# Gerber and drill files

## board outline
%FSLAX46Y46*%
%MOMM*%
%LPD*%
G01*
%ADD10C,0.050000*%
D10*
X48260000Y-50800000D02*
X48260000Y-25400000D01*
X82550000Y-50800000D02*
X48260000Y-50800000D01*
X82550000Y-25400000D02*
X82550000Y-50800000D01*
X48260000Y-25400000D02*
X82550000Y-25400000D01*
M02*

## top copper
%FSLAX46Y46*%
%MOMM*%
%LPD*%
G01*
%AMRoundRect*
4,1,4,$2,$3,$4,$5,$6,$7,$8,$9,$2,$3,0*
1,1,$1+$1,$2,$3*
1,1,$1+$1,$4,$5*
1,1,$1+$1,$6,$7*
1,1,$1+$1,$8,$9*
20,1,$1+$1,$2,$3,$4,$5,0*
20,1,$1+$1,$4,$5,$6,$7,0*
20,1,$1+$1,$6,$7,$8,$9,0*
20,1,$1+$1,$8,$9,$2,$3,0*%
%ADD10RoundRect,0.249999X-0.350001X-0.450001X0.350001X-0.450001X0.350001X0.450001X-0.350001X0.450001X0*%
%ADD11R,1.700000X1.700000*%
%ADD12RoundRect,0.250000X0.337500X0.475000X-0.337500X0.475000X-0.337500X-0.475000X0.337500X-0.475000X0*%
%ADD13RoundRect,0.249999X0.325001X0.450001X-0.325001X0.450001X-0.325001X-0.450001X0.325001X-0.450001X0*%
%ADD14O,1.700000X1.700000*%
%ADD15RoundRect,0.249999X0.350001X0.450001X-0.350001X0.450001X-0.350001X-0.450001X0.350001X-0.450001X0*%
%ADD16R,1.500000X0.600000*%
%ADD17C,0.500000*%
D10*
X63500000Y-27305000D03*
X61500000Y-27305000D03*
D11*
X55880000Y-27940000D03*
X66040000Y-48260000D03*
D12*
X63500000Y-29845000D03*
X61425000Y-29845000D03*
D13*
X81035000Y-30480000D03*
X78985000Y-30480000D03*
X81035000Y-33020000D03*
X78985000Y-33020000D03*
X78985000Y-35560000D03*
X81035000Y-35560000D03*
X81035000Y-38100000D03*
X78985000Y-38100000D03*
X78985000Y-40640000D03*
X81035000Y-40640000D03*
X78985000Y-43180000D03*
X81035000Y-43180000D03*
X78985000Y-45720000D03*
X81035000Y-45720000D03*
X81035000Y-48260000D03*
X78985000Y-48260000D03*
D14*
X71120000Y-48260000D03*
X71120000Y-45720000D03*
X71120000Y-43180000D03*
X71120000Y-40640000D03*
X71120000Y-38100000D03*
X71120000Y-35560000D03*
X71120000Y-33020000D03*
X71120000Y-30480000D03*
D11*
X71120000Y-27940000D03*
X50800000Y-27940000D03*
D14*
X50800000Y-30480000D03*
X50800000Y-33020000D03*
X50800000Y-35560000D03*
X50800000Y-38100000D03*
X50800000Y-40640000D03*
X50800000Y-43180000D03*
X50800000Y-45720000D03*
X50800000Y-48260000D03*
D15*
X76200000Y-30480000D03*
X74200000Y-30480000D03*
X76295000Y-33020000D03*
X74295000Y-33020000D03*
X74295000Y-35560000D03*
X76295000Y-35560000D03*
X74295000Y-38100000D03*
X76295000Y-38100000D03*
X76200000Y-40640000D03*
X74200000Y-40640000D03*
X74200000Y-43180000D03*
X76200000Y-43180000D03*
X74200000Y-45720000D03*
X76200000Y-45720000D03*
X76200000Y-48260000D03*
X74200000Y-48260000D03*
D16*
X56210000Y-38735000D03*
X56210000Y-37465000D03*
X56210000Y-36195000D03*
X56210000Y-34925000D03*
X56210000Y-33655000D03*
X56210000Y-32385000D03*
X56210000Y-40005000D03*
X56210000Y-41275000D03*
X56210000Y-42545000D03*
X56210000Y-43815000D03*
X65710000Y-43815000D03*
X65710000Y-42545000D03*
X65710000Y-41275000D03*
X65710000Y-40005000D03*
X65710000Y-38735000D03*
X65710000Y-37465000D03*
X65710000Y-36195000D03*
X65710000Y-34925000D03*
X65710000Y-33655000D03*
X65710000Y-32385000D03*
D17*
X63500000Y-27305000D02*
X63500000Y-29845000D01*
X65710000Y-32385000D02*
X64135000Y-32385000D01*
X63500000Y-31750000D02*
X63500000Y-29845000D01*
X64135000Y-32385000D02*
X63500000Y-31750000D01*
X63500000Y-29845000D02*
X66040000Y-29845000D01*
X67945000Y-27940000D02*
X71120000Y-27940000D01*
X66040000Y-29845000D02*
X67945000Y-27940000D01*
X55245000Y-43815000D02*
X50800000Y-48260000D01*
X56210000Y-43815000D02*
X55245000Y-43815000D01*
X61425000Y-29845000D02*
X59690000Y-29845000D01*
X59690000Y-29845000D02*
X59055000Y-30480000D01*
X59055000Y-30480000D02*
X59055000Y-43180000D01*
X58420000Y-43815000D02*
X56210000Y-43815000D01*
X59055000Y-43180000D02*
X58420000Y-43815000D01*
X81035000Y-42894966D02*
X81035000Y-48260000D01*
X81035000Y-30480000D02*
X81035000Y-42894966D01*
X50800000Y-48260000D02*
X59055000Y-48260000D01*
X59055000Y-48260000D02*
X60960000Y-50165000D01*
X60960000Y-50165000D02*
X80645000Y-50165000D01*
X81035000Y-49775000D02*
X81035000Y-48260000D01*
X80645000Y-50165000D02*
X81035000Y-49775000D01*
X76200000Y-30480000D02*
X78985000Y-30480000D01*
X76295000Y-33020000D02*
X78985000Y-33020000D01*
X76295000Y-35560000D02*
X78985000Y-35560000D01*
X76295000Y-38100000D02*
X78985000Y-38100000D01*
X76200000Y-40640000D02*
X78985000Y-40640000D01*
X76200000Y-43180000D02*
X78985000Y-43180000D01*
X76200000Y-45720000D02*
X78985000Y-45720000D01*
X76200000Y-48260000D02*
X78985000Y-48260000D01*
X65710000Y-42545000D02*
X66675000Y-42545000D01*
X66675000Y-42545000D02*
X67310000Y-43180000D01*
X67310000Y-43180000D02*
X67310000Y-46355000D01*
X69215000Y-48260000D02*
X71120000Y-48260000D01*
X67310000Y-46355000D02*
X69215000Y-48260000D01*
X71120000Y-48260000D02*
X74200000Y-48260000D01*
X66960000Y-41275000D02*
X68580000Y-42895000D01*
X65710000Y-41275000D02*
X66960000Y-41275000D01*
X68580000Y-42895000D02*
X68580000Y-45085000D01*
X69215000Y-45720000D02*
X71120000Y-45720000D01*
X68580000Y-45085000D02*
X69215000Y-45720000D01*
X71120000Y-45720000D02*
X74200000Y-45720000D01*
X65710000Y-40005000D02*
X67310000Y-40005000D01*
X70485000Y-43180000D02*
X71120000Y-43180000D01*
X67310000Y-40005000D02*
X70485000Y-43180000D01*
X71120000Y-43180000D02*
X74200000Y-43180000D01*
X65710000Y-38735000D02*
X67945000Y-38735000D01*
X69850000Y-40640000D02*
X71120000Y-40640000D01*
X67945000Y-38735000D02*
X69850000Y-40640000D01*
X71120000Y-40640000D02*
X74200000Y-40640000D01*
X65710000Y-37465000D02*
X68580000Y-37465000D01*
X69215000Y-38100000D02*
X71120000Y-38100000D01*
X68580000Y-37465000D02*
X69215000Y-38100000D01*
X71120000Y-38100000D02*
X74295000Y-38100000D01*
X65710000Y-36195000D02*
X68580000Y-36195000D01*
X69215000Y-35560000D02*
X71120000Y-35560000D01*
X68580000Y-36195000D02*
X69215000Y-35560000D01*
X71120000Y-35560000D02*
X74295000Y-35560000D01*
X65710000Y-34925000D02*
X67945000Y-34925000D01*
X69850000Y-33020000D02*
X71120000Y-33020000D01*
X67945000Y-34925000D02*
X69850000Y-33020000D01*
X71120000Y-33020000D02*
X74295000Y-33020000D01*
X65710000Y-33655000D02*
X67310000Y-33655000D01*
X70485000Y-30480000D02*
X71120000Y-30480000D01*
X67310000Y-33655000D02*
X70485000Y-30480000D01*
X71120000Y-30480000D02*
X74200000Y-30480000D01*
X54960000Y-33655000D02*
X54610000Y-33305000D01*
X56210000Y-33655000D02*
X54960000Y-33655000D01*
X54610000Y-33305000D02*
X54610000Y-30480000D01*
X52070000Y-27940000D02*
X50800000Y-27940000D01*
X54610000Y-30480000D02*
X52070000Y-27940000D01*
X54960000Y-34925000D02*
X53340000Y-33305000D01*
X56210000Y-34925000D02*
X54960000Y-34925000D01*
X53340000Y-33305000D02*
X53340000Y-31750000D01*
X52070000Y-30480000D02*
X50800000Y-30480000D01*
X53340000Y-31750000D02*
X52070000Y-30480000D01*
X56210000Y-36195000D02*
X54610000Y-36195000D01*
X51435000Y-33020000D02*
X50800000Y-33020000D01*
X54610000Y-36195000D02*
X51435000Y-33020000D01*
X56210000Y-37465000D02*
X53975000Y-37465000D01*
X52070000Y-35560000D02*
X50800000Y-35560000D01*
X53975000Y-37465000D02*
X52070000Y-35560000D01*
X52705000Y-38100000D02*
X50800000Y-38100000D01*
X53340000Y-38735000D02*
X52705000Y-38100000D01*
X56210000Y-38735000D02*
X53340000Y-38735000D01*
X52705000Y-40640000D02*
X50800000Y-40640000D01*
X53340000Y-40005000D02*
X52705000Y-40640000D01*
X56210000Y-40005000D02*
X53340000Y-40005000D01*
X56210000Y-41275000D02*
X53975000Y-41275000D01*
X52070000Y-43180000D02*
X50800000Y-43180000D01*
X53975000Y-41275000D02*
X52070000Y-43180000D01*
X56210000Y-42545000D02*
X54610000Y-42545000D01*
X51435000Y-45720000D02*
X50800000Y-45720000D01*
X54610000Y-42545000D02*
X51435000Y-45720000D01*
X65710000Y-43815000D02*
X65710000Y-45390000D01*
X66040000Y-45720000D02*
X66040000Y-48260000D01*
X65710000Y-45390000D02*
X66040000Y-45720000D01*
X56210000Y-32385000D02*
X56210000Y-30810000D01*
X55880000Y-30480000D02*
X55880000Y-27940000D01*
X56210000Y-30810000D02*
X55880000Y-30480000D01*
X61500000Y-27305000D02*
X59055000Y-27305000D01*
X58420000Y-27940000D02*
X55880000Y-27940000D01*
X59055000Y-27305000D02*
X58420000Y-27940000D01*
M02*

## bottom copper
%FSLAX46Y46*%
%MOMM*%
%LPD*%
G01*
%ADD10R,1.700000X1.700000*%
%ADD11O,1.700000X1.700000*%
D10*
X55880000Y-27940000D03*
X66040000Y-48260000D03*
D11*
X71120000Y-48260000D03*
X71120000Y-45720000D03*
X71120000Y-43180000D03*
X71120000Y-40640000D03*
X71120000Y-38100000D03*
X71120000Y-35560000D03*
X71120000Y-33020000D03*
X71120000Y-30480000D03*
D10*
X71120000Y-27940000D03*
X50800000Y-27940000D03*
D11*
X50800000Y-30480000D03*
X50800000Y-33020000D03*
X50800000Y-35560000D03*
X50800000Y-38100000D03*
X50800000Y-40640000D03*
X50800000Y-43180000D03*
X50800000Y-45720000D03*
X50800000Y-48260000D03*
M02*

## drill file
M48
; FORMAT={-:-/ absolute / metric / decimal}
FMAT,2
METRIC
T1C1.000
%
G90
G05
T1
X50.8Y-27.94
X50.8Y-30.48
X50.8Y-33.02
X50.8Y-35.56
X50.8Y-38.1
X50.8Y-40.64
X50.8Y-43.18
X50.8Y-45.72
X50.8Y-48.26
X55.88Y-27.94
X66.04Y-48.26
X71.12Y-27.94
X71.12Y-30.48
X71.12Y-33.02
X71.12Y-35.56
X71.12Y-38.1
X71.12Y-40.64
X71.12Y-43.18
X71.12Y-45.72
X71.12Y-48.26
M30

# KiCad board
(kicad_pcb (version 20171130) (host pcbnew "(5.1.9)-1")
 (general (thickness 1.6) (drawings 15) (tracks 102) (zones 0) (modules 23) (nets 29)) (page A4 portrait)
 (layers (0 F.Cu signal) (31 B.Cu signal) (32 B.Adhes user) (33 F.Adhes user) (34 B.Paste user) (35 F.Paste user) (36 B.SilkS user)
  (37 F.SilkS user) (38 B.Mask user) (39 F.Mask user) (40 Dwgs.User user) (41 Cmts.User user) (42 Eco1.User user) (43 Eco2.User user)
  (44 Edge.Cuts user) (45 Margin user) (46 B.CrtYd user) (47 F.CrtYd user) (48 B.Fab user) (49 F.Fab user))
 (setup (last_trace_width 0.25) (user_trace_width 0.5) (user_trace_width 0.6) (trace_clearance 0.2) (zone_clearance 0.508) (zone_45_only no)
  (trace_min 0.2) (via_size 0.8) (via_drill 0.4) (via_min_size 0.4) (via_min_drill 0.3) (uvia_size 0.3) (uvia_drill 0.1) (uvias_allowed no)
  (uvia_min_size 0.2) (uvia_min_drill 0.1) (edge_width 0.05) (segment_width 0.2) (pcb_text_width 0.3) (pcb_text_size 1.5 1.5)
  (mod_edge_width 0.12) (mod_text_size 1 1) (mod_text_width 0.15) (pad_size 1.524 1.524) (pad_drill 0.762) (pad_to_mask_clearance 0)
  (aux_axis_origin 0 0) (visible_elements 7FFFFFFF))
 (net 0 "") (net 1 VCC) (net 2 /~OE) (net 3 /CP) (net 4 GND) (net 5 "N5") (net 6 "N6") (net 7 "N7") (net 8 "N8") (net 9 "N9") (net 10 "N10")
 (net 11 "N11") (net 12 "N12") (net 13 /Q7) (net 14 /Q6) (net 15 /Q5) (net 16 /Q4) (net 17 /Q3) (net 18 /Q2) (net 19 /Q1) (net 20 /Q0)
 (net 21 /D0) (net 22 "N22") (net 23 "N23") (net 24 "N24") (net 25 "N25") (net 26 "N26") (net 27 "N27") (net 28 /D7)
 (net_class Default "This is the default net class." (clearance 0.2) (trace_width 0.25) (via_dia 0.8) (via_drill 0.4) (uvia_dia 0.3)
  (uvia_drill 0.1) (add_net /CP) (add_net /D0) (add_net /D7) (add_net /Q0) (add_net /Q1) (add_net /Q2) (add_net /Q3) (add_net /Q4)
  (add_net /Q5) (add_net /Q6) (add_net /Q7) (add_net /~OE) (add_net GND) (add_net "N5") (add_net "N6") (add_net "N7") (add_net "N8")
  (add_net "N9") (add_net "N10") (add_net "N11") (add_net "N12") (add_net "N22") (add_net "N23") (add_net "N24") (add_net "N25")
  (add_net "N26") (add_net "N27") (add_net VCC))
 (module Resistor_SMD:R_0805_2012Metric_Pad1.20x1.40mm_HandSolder (layer F.Cu) (at 62.5 27.305)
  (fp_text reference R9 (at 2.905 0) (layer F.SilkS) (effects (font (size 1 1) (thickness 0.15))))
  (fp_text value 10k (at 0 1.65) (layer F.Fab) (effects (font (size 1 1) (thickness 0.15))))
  (pad 2 smd roundrect (at 1 0) (size 1.2 1.4) (layers F.Cu F.Paste F.Mask) (roundrect_rratio 0.2083325) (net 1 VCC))
  (pad 1 smd roundrect (at -1 0) (size 1.2 1.4) (layers F.Cu F.Paste F.Mask) (roundrect_rratio 0.2083325) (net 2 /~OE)))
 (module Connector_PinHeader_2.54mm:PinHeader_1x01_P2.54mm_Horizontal (layer F.Cu) (at 55.88 27.94 90)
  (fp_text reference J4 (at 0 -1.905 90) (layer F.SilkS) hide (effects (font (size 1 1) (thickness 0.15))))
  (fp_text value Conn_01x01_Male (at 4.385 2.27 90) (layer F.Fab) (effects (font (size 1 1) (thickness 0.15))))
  (pad 1 thru_hole rect (at 0 0 90) (size 1.7 1.7) (drill 1) (layers *.Cu *.Mask) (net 2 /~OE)))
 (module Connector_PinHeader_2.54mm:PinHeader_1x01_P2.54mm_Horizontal (layer F.Cu) (at 66.04 48.26 270)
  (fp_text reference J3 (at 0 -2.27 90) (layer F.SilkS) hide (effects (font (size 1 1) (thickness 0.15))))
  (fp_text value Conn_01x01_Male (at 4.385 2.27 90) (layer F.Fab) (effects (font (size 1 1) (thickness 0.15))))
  (pad 1 thru_hole rect (at 0 0 270) (size 1.7 1.7) (drill 1) (layers *.Cu *.Mask) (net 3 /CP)))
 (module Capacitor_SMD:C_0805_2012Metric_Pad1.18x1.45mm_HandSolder (layer F.Cu) (at 62.4625 29.845 180)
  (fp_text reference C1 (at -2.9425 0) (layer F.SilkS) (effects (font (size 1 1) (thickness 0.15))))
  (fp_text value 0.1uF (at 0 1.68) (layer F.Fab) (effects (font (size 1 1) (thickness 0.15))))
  (pad 1 smd roundrect (at -1.0375 0 180) (size 1.175 1.45) (layers F.Cu F.Paste F.Mask) (roundrect_rratio 0.2127659574468085) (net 1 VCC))
  (pad 2 smd roundrect (at 1.0375 0 180) (size 1.175 1.45) (layers F.Cu F.Paste F.Mask) (roundrect_rratio 0.2127659574468085) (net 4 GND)))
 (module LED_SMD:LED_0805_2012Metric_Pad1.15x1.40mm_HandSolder (layer F.Cu) (at 80.01 30.48 180)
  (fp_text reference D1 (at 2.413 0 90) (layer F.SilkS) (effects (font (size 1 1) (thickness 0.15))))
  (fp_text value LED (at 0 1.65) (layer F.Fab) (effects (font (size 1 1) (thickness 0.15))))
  (pad 1 smd roundrect (at -1.025 0 180) (size 1.15 1.4) (layers F.Cu F.Paste F.Mask) (roundrect_rratio 0.2173904347826087) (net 4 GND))
  (pad 2 smd roundrect (at 1.025 0 180) (size 1.15 1.4) (layers F.Cu F.Paste F.Mask) (roundrect_rratio 0.2173904347826087) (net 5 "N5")))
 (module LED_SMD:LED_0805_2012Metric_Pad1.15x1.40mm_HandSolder (layer F.Cu) (at 80.01 33.02 180)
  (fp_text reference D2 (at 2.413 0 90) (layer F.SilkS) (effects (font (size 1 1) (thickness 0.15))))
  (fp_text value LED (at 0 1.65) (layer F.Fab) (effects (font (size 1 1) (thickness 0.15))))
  (pad 1 smd roundrect (at -1.025 0 180) (size 1.15 1.4) (layers F.Cu F.Paste F.Mask) (roundrect_rratio 0.2173904347826087) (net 4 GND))
  (pad 2 smd roundrect (at 1.025 0 180) (size 1.15 1.4) (layers F.Cu F.Paste F.Mask) (roundrect_rratio 0.2173904347826087) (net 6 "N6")))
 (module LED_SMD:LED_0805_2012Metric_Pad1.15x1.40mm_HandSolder (layer F.Cu) (at 80.01 35.56 180)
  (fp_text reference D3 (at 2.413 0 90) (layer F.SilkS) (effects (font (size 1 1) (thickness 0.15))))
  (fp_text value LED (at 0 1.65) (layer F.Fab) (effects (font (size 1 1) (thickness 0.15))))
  (pad 2 smd roundrect (at 1.025 0 180) (size 1.15 1.4) (layers F.Cu F.Paste F.Mask) (roundrect_rratio 0.2173904347826087) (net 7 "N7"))
  (pad 1 smd roundrect (at -1.025 0 180) (size 1.15 1.4) (layers F.Cu F.Paste F.Mask) (roundrect_rratio 0.2173904347826087) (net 4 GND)))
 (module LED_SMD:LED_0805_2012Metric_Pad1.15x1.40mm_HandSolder (layer F.Cu) (at 80.01 38.1 180)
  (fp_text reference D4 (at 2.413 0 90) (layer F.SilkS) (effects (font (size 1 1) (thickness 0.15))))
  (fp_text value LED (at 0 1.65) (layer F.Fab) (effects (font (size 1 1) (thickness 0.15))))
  (pad 1 smd roundrect (at -1.025 0 180) (size 1.15 1.4) (layers F.Cu F.Paste F.Mask) (roundrect_rratio 0.2173904347826087) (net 4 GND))
  (pad 2 smd roundrect (at 1.025 0 180) (size 1.15 1.4) (layers F.Cu F.Paste F.Mask) (roundrect_rratio 0.2173904347826087) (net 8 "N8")))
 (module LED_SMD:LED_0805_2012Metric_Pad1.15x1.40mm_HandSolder (layer F.Cu) (at 80.01 40.64 180)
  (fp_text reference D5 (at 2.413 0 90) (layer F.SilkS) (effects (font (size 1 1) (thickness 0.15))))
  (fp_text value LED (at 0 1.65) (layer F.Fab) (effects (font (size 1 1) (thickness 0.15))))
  (pad 2 smd roundrect (at 1.025 0 180) (size 1.15 1.4) (layers F.Cu F.Paste F.Mask) (roundrect_rratio 0.2173904347826087) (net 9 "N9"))
  (pad 1 smd roundrect (at -1.025 0 180) (size 1.15 1.4) (layers F.Cu F.Paste F.Mask) (roundrect_rratio 0.2173904347826087) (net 4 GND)))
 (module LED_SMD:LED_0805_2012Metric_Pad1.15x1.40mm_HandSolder (layer F.Cu) (at 80.01 43.18 180)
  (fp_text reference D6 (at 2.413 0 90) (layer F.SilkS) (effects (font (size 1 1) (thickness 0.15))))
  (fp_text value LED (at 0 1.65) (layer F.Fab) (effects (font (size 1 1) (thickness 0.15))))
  (pad 2 smd roundrect (at 1.025 0 180) (size 1.15 1.4) (layers F.Cu F.Paste F.Mask) (roundrect_rratio 0.2173904347826087) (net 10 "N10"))
  (pad 1 smd roundrect (at -1.025 0 180) (size 1.15 1.4) (layers F.Cu F.Paste F.Mask) (roundrect_rratio 0.2173904347826087) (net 4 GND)))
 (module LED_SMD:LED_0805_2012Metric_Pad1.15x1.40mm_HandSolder (layer F.Cu) (at 80.01 45.72 180)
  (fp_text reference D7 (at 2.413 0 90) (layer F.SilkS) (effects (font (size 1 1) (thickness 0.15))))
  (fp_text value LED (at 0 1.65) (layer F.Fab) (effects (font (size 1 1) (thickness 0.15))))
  (pad 2 smd roundrect (at 1.025 0 180) (size 1.15 1.4) (layers F.Cu F.Paste F.Mask) (roundrect_rratio 0.2173904347826087) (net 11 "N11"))
  (pad 1 smd roundrect (at -1.025 0 180) (size 1.15 1.4) (layers F.Cu F.Paste F.Mask) (roundrect_rratio 0.2173904347826087) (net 4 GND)))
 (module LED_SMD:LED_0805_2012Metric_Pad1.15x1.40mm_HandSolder (layer F.Cu) (at 80.01 48.26 180)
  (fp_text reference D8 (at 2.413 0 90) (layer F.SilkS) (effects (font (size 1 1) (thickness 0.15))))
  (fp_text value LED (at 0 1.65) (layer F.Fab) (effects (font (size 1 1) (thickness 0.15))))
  (pad 1 smd roundrect (at -1.025 0 180) (size 1.15 1.4) (layers F.Cu F.Paste F.Mask) (roundrect_rratio 0.2173904347826087) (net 4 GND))
  (pad 2 smd roundrect (at 1.025 0 180) (size 1.15 1.4) (layers F.Cu F.Paste F.Mask) (roundrect_rratio 0.2173904347826087) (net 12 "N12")))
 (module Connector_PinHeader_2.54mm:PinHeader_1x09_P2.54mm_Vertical (layer B.Cu) (at 71.12 27.94 180)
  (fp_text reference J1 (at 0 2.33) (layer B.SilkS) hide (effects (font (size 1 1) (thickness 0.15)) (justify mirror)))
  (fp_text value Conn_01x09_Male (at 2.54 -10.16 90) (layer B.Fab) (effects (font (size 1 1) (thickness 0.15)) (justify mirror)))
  (pad 9 thru_hole oval (at 0 -20.32 180) (size 1.7 1.7) (drill 1) (layers *.Cu *.Mask) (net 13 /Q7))
  (pad 8 thru_hole oval (at 0 -17.78 180) (size 1.7 1.7) (drill 1) (layers *.Cu *.Mask) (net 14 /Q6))
  (pad 7 thru_hole oval (at 0 -15.24 180) (size 1.7 1.7) (drill 1) (layers *.Cu *.Mask) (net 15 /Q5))
  (pad 6 thru_hole oval (at 0 -12.7 180) (size 1.7 1.7) (drill 1) (layers *.Cu *.Mask) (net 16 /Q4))
  (pad 5 thru_hole oval (at 0 -10.16 180) (size 1.7 1.7) (drill 1) (layers *.Cu *.Mask) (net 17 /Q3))
  (pad 4 thru_hole oval (at 0 -7.62 180) (size 1.7 1.7) (drill 1) (layers *.Cu *.Mask) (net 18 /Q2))
  (pad 3 thru_hole oval (at 0 -5.08 180) (size 1.7 1.7) (drill 1) (layers *.Cu *.Mask) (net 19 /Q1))
  (pad 2 thru_hole oval (at 0 -2.54 180) (size 1.7 1.7) (drill 1) (layers *.Cu *.Mask) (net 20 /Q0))
  (pad 1 thru_hole rect (at 0 0 180) (size 1.7 1.7) (drill 1) (layers *.Cu *.Mask) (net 1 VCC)))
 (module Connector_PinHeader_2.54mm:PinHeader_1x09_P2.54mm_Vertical (layer B.Cu) (at 50.8 27.94 180)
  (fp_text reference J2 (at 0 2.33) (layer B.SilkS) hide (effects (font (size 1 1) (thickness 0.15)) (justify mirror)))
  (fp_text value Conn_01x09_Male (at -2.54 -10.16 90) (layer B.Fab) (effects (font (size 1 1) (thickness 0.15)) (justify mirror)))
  (pad 1 thru_hole rect (at 0 0 180) (size 1.7 1.7) (drill 1) (layers *.Cu *.Mask) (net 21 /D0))
  (pad 2 thru_hole oval (at 0 -2.54 180) (size 1.7 1.7) (drill 1) (layers *.Cu *.Mask) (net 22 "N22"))
  (pad 3 thru_hole oval (at 0 -5.08 180) (size 1.7 1.7) (drill 1) (layers *.Cu *.Mask) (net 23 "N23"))
  (pad 4 thru_hole oval (at 0 -7.62 180) (size 1.7 1.7) (drill 1) (layers *.Cu *.Mask) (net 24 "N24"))
  (pad 5 thru_hole oval (at 0 -10.16 180) (size 1.7 1.7) (drill 1) (layers *.Cu *.Mask) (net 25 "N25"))
  (pad 6 thru_hole oval (at 0 -12.7 180) (size 1.7 1.7) (drill 1) (layers *.Cu *.Mask) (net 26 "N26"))
  (pad 7 thru_hole oval (at 0 -15.24 180) (size 1.7 1.7) (drill 1) (layers *.Cu *.Mask) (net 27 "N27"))
  (pad 8 thru_hole oval (at 0 -17.78 180) (size 1.7 1.7) (drill 1) (layers *.Cu *.Mask) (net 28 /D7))
  (pad 9 thru_hole oval (at 0 -20.32 180) (size 1.7 1.7) (drill 1) (layers *.Cu *.Mask) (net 4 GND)))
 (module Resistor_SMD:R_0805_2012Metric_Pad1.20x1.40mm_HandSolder (layer F.Cu) (at 75.2 30.48 180)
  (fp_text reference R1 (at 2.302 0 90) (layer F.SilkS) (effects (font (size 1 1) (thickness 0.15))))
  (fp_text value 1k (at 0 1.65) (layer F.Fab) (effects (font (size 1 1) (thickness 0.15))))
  (pad 1 smd roundrect (at -1 0 180) (size 1.2 1.4) (layers F.Cu F.Paste F.Mask) (roundrect_rratio 0.2083325) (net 5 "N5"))
  (pad 2 smd roundrect (at 1 0 180) (size 1.2 1.4) (layers F.Cu F.Paste F.Mask) (roundrect_rratio 0.2083325) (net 20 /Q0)))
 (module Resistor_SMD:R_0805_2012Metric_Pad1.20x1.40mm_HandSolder (layer F.Cu) (at 75.295 33.02 180)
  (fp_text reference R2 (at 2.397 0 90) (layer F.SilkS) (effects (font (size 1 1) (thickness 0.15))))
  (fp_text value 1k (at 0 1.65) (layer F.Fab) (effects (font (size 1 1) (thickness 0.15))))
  (pad 1 smd roundrect (at -1 0 180) (size 1.2 1.4) (layers F.Cu F.Paste F.Mask) (roundrect_rratio 0.2083325) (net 6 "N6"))
  (pad 2 smd roundrect (at 1 0 180) (size 1.2 1.4) (layers F.Cu F.Paste F.Mask) (roundrect_rratio 0.2083325) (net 19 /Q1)))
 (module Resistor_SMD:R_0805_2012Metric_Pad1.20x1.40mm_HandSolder (layer F.Cu) (at 75.295 35.56 180)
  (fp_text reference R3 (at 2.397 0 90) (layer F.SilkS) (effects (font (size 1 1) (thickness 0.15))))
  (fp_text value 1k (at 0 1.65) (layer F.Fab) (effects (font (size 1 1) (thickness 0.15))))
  (pad 2 smd roundrect (at 1 0 180) (size 1.2 1.4) (layers F.Cu F.Paste F.Mask) (roundrect_rratio 0.2083325) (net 18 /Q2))
  (pad 1 smd roundrect (at -1 0 180) (size 1.2 1.4) (layers F.Cu F.Paste F.Mask) (roundrect_rratio 0.2083325) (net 7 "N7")))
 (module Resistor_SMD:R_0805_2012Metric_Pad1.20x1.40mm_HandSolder (layer F.Cu) (at 75.295 38.1 180)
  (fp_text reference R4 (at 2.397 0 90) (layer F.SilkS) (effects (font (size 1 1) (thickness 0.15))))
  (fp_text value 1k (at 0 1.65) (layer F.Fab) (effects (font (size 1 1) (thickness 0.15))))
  (pad 2 smd roundrect (at 1 0 180) (size 1.2 1.4) (layers F.Cu F.Paste F.Mask) (roundrect_rratio 0.2083325) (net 17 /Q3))
  (pad 1 smd roundrect (at -1 0 180) (size 1.2 1.4) (layers F.Cu F.Paste F.Mask) (roundrect_rratio 0.2083325) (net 8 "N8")))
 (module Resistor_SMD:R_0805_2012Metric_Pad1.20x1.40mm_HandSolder (layer F.Cu) (at 75.2 40.64 180)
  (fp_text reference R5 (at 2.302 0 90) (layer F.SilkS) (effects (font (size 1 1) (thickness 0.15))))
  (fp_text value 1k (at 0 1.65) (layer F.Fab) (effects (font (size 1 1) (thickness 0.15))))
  (pad 1 smd roundrect (at -1 0 180) (size 1.2 1.4) (layers F.Cu F.Paste F.Mask) (roundrect_rratio 0.2083325) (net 9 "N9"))
  (pad 2 smd roundrect (at 1 0 180) (size 1.2 1.4) (layers F.Cu F.Paste F.Mask) (roundrect_rratio 0.2083325) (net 16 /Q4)))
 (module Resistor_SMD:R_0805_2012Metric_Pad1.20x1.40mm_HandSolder (layer F.Cu) (at 75.2 43.18 180)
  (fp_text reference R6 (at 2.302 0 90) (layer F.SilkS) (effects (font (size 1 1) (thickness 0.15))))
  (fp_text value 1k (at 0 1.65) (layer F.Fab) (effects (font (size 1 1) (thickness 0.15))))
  (pad 2 smd roundrect (at 1 0 180) (size 1.2 1.4) (layers F.Cu F.Paste F.Mask) (roundrect_rratio 0.2083325) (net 15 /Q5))
  (pad 1 smd roundrect (at -1 0 180) (size 1.2 1.4) (layers F.Cu F.Paste F.Mask) (roundrect_rratio 0.2083325) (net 10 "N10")))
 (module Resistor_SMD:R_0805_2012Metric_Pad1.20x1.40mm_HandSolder (layer F.Cu) (at 75.2 45.72 180)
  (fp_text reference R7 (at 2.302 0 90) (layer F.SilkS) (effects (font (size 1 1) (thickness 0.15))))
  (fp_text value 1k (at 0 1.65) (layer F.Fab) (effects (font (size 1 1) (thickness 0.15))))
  (pad 2 smd roundrect (at 1 0 180) (size 1.2 1.4) (layers F.Cu F.Paste F.Mask) (roundrect_rratio 0.2083325) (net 14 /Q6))
  (pad 1 smd roundrect (at -1 0 180) (size 1.2 1.4) (layers F.Cu F.Paste F.Mask) (roundrect_rratio 0.2083325) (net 11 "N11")))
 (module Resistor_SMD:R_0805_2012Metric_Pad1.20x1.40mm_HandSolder (layer F.Cu) (at 75.2 48.26 180)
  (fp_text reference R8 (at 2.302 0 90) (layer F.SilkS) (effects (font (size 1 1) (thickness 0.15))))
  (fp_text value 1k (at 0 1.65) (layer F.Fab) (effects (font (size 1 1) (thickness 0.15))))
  (pad 1 smd roundrect (at -1 0 180) (size 1.2 1.4) (layers F.Cu F.Paste F.Mask) (roundrect_rratio 0.2083325) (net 12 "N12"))
  (pad 2 smd roundrect (at 1 0 180) (size 1.2 1.4) (layers F.Cu F.Paste F.Mask) (roundrect_rratio 0.2083325) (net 13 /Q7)))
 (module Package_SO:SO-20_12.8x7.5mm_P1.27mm (layer F.Cu) (at 60.96 38.1)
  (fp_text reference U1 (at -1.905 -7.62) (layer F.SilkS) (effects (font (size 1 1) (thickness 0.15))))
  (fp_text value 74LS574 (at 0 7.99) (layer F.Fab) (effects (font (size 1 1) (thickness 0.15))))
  (pad 6 smd rect (at -4.75 0.635) (size 1.5 0.6) (layers F.Cu F.Paste F.Mask) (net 25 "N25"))
  (pad 5 smd rect (at -4.75 -0.635) (size 1.5 0.6) (layers F.Cu F.Paste F.Mask) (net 24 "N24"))
  (pad 4 smd rect (at -4.75 -1.905) (size 1.5 0.6) (layers F.Cu F.Paste F.Mask) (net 23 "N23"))
  (pad 3 smd rect (at -4.75 -3.175) (size 1.5 0.6) (layers F.Cu F.Paste F.Mask) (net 22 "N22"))
  (pad 2 smd rect (at -4.75 -4.445) (size 1.5 0.6) (layers F.Cu F.Paste F.Mask) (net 21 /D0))
  (pad 1 smd rect (at -4.75 -5.715) (size 1.5 0.6) (layers F.Cu F.Paste F.Mask) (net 2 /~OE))
  (pad 7 smd rect (at -4.75 1.905) (size 1.5 0.6) (layers F.Cu F.Paste F.Mask) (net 26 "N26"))
  (pad 8 smd rect (at -4.75 3.175) (size 1.5 0.6) (layers F.Cu F.Paste F.Mask) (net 27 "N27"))
  (pad 9 smd rect (at -4.75 4.445) (size 1.5 0.6) (layers F.Cu F.Paste F.Mask) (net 28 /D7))
  (pad 10 smd rect (at -4.75 5.715) (size 1.5 0.6) (layers F.Cu F.Paste F.Mask) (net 4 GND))
  (pad 11 smd rect (at 4.75 5.715) (size 1.5 0.6) (layers F.Cu F.Paste F.Mask) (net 3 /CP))
  (pad 12 smd rect (at 4.75 4.445) (size 1.5 0.6) (layers F.Cu F.Paste F.Mask) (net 13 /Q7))
  (pad 13 smd rect (at 4.75 3.175) (size 1.5 0.6) (layers F.Cu F.Paste F.Mask) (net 14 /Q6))
  (pad 14 smd rect (at 4.75 1.905) (size 1.5 0.6) (layers F.Cu F.Paste F.Mask) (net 15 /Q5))
  (pad 15 smd rect (at 4.75 0.635) (size 1.5 0.6) (layers F.Cu F.Paste F.Mask) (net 16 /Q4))
  (pad 16 smd rect (at 4.75 -0.635) (size 1.5 0.6) (layers F.Cu F.Paste F.Mask) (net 17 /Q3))
  (pad 17 smd rect (at 4.75 -1.905) (size 1.5 0.6) (layers F.Cu F.Paste F.Mask) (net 18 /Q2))
  (pad 18 smd rect (at 4.75 -3.175) (size 1.5 0.6) (layers F.Cu F.Paste F.Mask) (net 19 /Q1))
  (pad 19 smd rect (at 4.75 -4.445) (size 1.5 0.6) (layers F.Cu F.Paste F.Mask) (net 20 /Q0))
  (pad 20 smd rect (at 4.75 -5.715) (size 1.5 0.6) (layers F.Cu F.Paste F.Mask) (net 1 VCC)))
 (gr_line (start 48.26 50.8) (end 48.26 25.4) (layer Edge.Cuts) (width 0.05))
 (gr_line (start 82.55 50.8) (end 48.26 50.8) (layer Edge.Cuts) (width 0.05))
 (gr_line (start 82.55 25.4) (end 82.55 50.8) (layer Edge.Cuts) (width 0.05))
 (gr_line (start 48.26 25.4) (end 82.55 25.4) (layer Edge.Cuts) (width 0.05))
 (segment (start 63.5 27.305) (end 63.5 29.845) (width 0.5) (layer F.Cu) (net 1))
 (segment (start 65.71 32.385) (end 64.135 32.385) (width 0.5) (layer F.Cu) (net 1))
 (segment (start 63.5 31.75) (end 63.5 29.845) (width 0.5) (layer F.Cu) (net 1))
 (segment (start 64.135 32.385) (end 63.5 31.75) (width 0.5) (layer F.Cu) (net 1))
 (segment (start 63.5 29.845) (end 66.04 29.845) (width 0.5) (layer F.Cu) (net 1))
 (segment (start 67.945 27.94) (end 71.12 27.94) (width 0.5) (layer F.Cu) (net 1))
 (segment (start 66.04 29.845) (end 67.945 27.94) (width 0.5) (layer F.Cu) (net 1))
 (segment (start 55.245 43.815) (end 50.8 48.26) (width 0.5) (layer F.Cu) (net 4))
 (segment (start 56.21 43.815) (end 55.245 43.815) (width 0.5) (layer F.Cu) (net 4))
 (segment (start 61.425 29.845) (end 59.69 29.845) (width 0.5) (layer F.Cu) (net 4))
 (segment (start 59.69 29.845) (end 59.055 30.48) (width 0.5) (layer F.Cu) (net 4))
 (segment (start 59.055 30.48) (end 59.055 43.18) (width 0.5) (layer F.Cu) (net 4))
 (segment (start 58.42 43.815) (end 56.21 43.815) (width 0.5) (layer F.Cu) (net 4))
 (segment (start 59.055 43.18) (end 58.42 43.815) (width 0.5) (layer F.Cu) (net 4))
 (segment (start 81.035 42.894966) (end 81.035 48.26) (width 0.5) (layer F.Cu) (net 4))
 (segment (start 81.035 30.48) (end 81.035 42.894966) (width 0.5) (layer F.Cu) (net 4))
 (segment (start 50.8 48.26) (end 59.055 48.26) (width 0.5) (layer F.Cu) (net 4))
 (segment (start 59.055 48.26) (end 60.96 50.165) (width 0.5) (layer F.Cu) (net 4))
 (segment (start 60.96 50.165) (end 80.645 50.165) (width 0.5) (layer F.Cu) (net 4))
 (segment (start 81.035 49.775) (end 81.035 48.26) (width 0.5) (layer F.Cu) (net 4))
 (segment (start 80.645 50.165) (end 81.035 49.775) (width 0.5) (layer F.Cu) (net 4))
 (segment (start 76.2 30.48) (end 78.985 30.48) (width 0.5) (layer F.Cu) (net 5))
 (segment (start 76.295 33.02) (end 78.985 33.02) (width 0.5) (layer F.Cu) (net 6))
 (segment (start 76.295 35.56) (end 78.985 35.56) (width 0.5) (layer F.Cu) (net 7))
 (segment (start 76.295 38.1) (end 78.985 38.1) (width 0.5) (layer F.Cu) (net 8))
 (segment (start 76.2 40.64) (end 78.985 40.64) (width 0.5) (layer F.Cu) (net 9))
 (segment (start 76.2 43.18) (end 78.985 43.18) (width 0.5) (layer F.Cu) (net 10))
 (segment (start 76.2 45.72) (end 78.985 45.72) (width 0.5) (layer F.Cu) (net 11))
 (segment (start 76.2 48.26) (end 78.985 48.26) (width 0.5) (layer F.Cu) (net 12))
 (segment (start 65.71 42.545) (end 66.675 42.545) (width 0.5) (layer F.Cu) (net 13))
 (segment (start 66.675 42.545) (end 67.31 43.18) (width 0.5) (layer F.Cu) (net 13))
 (segment (start 67.31 43.18) (end 67.31 46.355) (width 0.5) (layer F.Cu) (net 13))
 (segment (start 69.215 48.26) (end 71.12 48.26) (width 0.5) (layer F.Cu) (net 13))
 (segment (start 67.31 46.355) (end 69.215 48.26) (width 0.5) (layer F.Cu) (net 13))
 (segment (start 71.12 48.26) (end 74.2 48.26) (width 0.5) (layer F.Cu) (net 13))
 (segment (start 66.96 41.275) (end 68.58 42.895) (width 0.5) (layer F.Cu) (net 14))
 (segment (start 65.71 41.275) (end 66.96 41.275) (width 0.5) (layer F.Cu) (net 14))
 (segment (start 68.58 42.895) (end 68.58 45.085) (width 0.5) (layer F.Cu) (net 14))
 (segment (start 69.215 45.72) (end 71.12 45.72) (width 0.5) (layer F.Cu) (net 14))
 (segment (start 68.58 45.085) (end 69.215 45.72) (width 0.5) (layer F.Cu) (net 14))
 (segment (start 71.12 45.72) (end 74.2 45.72) (width 0.5) (layer F.Cu) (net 14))
 (segment (start 65.71 40.005) (end 67.31 40.005) (width 0.5) (layer F.Cu) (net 15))
 (segment (start 70.485 43.18) (end 71.12 43.18) (width 0.5) (layer F.Cu) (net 15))
 (segment (start 67.31 40.005) (end 70.485 43.18) (width 0.5) (layer F.Cu) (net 15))
 (segment (start 71.12 43.18) (end 74.2 43.18) (width 0.5) (layer F.Cu) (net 15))
 (segment (start 65.71 38.735) (end 67.945 38.735) (width 0.5) (layer F.Cu) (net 16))
 (segment (start 69.85 40.64) (end 71.12 40.64) (width 0.5) (layer F.Cu) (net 16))
 (segment (start 67.945 38.735) (end 69.85 40.64) (width 0.5) (layer F.Cu) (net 16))
 (segment (start 71.12 40.64) (end 74.2 40.64) (width 0.5) (layer F.Cu) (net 16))
 (segment (start 65.71 37.465) (end 68.58 37.465) (width 0.5) (layer F.Cu) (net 17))
 (segment (start 69.215 38.1) (end 71.12 38.1) (width 0.5) (layer F.Cu) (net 17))
 (segment (start 68.58 37.465) (end 69.215 38.1) (width 0.5) (layer F.Cu) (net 17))
 (segment (start 71.12 38.1) (end 74.295 38.1) (width 0.5) (layer F.Cu) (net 17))
 (segment (start 65.71 36.195) (end 68.58 36.195) (width 0.5) (layer F.Cu) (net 18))
 (segment (start 69.215 35.56) (end 71.12 35.56) (width 0.5) (layer F.Cu) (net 18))
 (segment (start 68.58 36.195) (end 69.215 35.56) (width 0.5) (layer F.Cu) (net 18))
 (segment (start 71.12 35.56) (end 74.295 35.56) (width 0.5) (layer F.Cu) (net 18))
 (segment (start 65.71 34.925) (end 67.945 34.925) (width 0.5) (layer F.Cu) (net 19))
 (segment (start 69.85 33.02) (end 71.12 33.02) (width 0.5) (layer F.Cu) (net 19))
 (segment (start 67.945 34.925) (end 69.85 33.02) (width 0.5) (layer F.Cu) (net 19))
 (segment (start 71.12 33.02) (end 74.295 33.02) (width 0.5) (layer F.Cu) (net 19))
 (segment (start 65.71 33.655) (end 67.31 33.655) (width 0.5) (layer F.Cu) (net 20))
 (segment (start 70.485 30.48) (end 71.12 30.48) (width 0.5) (layer F.Cu) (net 20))
 (segment (start 67.31 33.655) (end 70.485 30.48) (width 0.5) (layer F.Cu) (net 20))
 (segment (start 71.12 30.48) (end 74.2 30.48) (width 0.5) (layer F.Cu) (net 20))
 (segment (start 54.96 33.655) (end 54.61 33.305) (width 0.5) (layer F.Cu) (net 21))
 (segment (start 56.21 33.655) (end 54.96 33.655) (width 0.5) (layer F.Cu) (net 21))
 (segment (start 54.61 33.305) (end 54.61 30.48) (width 0.5) (layer F.Cu) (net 21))
 (segment (start 52.07 27.94) (end 50.8 27.94) (width 0.5) (layer F.Cu) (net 21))
 (segment (start 54.61 30.48) (end 52.07 27.94) (width 0.5) (layer F.Cu) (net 21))
 (segment (start 54.96 34.925) (end 53.34 33.305) (width 0.5) (layer F.Cu) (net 22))
 (segment (start 56.21 34.925) (end 54.96 34.925) (width 0.5) (layer F.Cu) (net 22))
 (segment (start 53.34 33.305) (end 53.34 31.75) (width 0.5) (layer F.Cu) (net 22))
 (segment (start 52.07 30.48) (end 50.8 30.48) (width 0.5) (layer F.Cu) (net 22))
 (segment (start 53.34 31.75) (end 52.07 30.48) (width 0.5) (layer F.Cu) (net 22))
 (segment (start 56.21 36.195) (end 54.61 36.195) (width 0.5) (layer F.Cu) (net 23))
 (segment (start 51.435 33.02) (end 50.8 33.02) (width 0.5) (layer F.Cu) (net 23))
 (segment (start 54.61 36.195) (end 51.435 33.02) (width 0.5) (layer F.Cu) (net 23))
 (segment (start 56.21 37.465) (end 53.975 37.465) (width 0.5) (layer F.Cu) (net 24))
 (segment (start 52.07 35.56) (end 50.8 35.56) (width 0.5) (layer F.Cu) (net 24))
 (segment (start 53.975 37.465) (end 52.07 35.56) (width 0.5) (layer F.Cu) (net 24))
 (segment (start 52.705 38.1) (end 50.8 38.1) (width 0.5) (layer F.Cu) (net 25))
 (segment (start 53.34 38.735) (end 52.705 38.1) (width 0.5) (layer F.Cu) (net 25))
 (segment (start 56.21 38.735) (end 53.34 38.735) (width 0.5) (layer F.Cu) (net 25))
 (segment (start 52.705 40.64) (end 50.8 40.64) (width 0.5) (layer F.Cu) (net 26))
 (segment (start 53.34 40.005) (end 52.705 40.64) (width 0.5) (layer F.Cu) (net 26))
 (segment (start 56.21 40.005) (end 53.34 40.005) (width 0.5) (layer F.Cu) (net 26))
 (segment (start 56.21 41.275) (end 53.975 41.275) (width 0.5) (layer F.Cu) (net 27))
 (segment (start 52.07 43.18) (end 50.8 43.18) (width 0.5) (layer F.Cu) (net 27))
 (segment (start 53.975 41.275) (end 52.07 43.18) (width 0.5) (layer F.Cu) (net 27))
 (segment (start 56.21 42.545) (end 54.61 42.545) (width 0.5) (layer F.Cu) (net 28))
 (segment (start 51.435 45.72) (end 50.8 45.72) (width 0.5) (layer F.Cu) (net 28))
 (segment (start 54.61 42.545) (end 51.435 45.72) (width 0.5) (layer F.Cu) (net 28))
 (segment (start 65.71 43.815) (end 65.71 45.39) (width 0.5) (layer F.Cu) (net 3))
 (segment (start 66.04 45.72) (end 66.04 48.26) (width 0.5) (layer F.Cu) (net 3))
 (segment (start 65.71 45.39) (end 66.04 45.72) (width 0.5) (layer F.Cu) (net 3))
 (segment (start 56.21 32.385) (end 56.21 30.81) (width 0.5) (layer F.Cu) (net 2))
 (segment (start 55.88 30.48) (end 55.88 27.94) (width 0.5) (layer F.Cu) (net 2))
 (segment (start 56.21 30.81) (end 55.88 30.48) (width 0.5) (layer F.Cu) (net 2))
 (segment (start 61.5 27.305) (end 59.055 27.305) (width 0.5) (layer F.Cu) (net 2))
 (segment (start 58.42 27.94) (end 55.88 27.94) (width 0.5) (layer F.Cu) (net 2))
 (segment (start 59.055 27.305) (end 58.42 27.94) (width 0.5) (layer F.Cu) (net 2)))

